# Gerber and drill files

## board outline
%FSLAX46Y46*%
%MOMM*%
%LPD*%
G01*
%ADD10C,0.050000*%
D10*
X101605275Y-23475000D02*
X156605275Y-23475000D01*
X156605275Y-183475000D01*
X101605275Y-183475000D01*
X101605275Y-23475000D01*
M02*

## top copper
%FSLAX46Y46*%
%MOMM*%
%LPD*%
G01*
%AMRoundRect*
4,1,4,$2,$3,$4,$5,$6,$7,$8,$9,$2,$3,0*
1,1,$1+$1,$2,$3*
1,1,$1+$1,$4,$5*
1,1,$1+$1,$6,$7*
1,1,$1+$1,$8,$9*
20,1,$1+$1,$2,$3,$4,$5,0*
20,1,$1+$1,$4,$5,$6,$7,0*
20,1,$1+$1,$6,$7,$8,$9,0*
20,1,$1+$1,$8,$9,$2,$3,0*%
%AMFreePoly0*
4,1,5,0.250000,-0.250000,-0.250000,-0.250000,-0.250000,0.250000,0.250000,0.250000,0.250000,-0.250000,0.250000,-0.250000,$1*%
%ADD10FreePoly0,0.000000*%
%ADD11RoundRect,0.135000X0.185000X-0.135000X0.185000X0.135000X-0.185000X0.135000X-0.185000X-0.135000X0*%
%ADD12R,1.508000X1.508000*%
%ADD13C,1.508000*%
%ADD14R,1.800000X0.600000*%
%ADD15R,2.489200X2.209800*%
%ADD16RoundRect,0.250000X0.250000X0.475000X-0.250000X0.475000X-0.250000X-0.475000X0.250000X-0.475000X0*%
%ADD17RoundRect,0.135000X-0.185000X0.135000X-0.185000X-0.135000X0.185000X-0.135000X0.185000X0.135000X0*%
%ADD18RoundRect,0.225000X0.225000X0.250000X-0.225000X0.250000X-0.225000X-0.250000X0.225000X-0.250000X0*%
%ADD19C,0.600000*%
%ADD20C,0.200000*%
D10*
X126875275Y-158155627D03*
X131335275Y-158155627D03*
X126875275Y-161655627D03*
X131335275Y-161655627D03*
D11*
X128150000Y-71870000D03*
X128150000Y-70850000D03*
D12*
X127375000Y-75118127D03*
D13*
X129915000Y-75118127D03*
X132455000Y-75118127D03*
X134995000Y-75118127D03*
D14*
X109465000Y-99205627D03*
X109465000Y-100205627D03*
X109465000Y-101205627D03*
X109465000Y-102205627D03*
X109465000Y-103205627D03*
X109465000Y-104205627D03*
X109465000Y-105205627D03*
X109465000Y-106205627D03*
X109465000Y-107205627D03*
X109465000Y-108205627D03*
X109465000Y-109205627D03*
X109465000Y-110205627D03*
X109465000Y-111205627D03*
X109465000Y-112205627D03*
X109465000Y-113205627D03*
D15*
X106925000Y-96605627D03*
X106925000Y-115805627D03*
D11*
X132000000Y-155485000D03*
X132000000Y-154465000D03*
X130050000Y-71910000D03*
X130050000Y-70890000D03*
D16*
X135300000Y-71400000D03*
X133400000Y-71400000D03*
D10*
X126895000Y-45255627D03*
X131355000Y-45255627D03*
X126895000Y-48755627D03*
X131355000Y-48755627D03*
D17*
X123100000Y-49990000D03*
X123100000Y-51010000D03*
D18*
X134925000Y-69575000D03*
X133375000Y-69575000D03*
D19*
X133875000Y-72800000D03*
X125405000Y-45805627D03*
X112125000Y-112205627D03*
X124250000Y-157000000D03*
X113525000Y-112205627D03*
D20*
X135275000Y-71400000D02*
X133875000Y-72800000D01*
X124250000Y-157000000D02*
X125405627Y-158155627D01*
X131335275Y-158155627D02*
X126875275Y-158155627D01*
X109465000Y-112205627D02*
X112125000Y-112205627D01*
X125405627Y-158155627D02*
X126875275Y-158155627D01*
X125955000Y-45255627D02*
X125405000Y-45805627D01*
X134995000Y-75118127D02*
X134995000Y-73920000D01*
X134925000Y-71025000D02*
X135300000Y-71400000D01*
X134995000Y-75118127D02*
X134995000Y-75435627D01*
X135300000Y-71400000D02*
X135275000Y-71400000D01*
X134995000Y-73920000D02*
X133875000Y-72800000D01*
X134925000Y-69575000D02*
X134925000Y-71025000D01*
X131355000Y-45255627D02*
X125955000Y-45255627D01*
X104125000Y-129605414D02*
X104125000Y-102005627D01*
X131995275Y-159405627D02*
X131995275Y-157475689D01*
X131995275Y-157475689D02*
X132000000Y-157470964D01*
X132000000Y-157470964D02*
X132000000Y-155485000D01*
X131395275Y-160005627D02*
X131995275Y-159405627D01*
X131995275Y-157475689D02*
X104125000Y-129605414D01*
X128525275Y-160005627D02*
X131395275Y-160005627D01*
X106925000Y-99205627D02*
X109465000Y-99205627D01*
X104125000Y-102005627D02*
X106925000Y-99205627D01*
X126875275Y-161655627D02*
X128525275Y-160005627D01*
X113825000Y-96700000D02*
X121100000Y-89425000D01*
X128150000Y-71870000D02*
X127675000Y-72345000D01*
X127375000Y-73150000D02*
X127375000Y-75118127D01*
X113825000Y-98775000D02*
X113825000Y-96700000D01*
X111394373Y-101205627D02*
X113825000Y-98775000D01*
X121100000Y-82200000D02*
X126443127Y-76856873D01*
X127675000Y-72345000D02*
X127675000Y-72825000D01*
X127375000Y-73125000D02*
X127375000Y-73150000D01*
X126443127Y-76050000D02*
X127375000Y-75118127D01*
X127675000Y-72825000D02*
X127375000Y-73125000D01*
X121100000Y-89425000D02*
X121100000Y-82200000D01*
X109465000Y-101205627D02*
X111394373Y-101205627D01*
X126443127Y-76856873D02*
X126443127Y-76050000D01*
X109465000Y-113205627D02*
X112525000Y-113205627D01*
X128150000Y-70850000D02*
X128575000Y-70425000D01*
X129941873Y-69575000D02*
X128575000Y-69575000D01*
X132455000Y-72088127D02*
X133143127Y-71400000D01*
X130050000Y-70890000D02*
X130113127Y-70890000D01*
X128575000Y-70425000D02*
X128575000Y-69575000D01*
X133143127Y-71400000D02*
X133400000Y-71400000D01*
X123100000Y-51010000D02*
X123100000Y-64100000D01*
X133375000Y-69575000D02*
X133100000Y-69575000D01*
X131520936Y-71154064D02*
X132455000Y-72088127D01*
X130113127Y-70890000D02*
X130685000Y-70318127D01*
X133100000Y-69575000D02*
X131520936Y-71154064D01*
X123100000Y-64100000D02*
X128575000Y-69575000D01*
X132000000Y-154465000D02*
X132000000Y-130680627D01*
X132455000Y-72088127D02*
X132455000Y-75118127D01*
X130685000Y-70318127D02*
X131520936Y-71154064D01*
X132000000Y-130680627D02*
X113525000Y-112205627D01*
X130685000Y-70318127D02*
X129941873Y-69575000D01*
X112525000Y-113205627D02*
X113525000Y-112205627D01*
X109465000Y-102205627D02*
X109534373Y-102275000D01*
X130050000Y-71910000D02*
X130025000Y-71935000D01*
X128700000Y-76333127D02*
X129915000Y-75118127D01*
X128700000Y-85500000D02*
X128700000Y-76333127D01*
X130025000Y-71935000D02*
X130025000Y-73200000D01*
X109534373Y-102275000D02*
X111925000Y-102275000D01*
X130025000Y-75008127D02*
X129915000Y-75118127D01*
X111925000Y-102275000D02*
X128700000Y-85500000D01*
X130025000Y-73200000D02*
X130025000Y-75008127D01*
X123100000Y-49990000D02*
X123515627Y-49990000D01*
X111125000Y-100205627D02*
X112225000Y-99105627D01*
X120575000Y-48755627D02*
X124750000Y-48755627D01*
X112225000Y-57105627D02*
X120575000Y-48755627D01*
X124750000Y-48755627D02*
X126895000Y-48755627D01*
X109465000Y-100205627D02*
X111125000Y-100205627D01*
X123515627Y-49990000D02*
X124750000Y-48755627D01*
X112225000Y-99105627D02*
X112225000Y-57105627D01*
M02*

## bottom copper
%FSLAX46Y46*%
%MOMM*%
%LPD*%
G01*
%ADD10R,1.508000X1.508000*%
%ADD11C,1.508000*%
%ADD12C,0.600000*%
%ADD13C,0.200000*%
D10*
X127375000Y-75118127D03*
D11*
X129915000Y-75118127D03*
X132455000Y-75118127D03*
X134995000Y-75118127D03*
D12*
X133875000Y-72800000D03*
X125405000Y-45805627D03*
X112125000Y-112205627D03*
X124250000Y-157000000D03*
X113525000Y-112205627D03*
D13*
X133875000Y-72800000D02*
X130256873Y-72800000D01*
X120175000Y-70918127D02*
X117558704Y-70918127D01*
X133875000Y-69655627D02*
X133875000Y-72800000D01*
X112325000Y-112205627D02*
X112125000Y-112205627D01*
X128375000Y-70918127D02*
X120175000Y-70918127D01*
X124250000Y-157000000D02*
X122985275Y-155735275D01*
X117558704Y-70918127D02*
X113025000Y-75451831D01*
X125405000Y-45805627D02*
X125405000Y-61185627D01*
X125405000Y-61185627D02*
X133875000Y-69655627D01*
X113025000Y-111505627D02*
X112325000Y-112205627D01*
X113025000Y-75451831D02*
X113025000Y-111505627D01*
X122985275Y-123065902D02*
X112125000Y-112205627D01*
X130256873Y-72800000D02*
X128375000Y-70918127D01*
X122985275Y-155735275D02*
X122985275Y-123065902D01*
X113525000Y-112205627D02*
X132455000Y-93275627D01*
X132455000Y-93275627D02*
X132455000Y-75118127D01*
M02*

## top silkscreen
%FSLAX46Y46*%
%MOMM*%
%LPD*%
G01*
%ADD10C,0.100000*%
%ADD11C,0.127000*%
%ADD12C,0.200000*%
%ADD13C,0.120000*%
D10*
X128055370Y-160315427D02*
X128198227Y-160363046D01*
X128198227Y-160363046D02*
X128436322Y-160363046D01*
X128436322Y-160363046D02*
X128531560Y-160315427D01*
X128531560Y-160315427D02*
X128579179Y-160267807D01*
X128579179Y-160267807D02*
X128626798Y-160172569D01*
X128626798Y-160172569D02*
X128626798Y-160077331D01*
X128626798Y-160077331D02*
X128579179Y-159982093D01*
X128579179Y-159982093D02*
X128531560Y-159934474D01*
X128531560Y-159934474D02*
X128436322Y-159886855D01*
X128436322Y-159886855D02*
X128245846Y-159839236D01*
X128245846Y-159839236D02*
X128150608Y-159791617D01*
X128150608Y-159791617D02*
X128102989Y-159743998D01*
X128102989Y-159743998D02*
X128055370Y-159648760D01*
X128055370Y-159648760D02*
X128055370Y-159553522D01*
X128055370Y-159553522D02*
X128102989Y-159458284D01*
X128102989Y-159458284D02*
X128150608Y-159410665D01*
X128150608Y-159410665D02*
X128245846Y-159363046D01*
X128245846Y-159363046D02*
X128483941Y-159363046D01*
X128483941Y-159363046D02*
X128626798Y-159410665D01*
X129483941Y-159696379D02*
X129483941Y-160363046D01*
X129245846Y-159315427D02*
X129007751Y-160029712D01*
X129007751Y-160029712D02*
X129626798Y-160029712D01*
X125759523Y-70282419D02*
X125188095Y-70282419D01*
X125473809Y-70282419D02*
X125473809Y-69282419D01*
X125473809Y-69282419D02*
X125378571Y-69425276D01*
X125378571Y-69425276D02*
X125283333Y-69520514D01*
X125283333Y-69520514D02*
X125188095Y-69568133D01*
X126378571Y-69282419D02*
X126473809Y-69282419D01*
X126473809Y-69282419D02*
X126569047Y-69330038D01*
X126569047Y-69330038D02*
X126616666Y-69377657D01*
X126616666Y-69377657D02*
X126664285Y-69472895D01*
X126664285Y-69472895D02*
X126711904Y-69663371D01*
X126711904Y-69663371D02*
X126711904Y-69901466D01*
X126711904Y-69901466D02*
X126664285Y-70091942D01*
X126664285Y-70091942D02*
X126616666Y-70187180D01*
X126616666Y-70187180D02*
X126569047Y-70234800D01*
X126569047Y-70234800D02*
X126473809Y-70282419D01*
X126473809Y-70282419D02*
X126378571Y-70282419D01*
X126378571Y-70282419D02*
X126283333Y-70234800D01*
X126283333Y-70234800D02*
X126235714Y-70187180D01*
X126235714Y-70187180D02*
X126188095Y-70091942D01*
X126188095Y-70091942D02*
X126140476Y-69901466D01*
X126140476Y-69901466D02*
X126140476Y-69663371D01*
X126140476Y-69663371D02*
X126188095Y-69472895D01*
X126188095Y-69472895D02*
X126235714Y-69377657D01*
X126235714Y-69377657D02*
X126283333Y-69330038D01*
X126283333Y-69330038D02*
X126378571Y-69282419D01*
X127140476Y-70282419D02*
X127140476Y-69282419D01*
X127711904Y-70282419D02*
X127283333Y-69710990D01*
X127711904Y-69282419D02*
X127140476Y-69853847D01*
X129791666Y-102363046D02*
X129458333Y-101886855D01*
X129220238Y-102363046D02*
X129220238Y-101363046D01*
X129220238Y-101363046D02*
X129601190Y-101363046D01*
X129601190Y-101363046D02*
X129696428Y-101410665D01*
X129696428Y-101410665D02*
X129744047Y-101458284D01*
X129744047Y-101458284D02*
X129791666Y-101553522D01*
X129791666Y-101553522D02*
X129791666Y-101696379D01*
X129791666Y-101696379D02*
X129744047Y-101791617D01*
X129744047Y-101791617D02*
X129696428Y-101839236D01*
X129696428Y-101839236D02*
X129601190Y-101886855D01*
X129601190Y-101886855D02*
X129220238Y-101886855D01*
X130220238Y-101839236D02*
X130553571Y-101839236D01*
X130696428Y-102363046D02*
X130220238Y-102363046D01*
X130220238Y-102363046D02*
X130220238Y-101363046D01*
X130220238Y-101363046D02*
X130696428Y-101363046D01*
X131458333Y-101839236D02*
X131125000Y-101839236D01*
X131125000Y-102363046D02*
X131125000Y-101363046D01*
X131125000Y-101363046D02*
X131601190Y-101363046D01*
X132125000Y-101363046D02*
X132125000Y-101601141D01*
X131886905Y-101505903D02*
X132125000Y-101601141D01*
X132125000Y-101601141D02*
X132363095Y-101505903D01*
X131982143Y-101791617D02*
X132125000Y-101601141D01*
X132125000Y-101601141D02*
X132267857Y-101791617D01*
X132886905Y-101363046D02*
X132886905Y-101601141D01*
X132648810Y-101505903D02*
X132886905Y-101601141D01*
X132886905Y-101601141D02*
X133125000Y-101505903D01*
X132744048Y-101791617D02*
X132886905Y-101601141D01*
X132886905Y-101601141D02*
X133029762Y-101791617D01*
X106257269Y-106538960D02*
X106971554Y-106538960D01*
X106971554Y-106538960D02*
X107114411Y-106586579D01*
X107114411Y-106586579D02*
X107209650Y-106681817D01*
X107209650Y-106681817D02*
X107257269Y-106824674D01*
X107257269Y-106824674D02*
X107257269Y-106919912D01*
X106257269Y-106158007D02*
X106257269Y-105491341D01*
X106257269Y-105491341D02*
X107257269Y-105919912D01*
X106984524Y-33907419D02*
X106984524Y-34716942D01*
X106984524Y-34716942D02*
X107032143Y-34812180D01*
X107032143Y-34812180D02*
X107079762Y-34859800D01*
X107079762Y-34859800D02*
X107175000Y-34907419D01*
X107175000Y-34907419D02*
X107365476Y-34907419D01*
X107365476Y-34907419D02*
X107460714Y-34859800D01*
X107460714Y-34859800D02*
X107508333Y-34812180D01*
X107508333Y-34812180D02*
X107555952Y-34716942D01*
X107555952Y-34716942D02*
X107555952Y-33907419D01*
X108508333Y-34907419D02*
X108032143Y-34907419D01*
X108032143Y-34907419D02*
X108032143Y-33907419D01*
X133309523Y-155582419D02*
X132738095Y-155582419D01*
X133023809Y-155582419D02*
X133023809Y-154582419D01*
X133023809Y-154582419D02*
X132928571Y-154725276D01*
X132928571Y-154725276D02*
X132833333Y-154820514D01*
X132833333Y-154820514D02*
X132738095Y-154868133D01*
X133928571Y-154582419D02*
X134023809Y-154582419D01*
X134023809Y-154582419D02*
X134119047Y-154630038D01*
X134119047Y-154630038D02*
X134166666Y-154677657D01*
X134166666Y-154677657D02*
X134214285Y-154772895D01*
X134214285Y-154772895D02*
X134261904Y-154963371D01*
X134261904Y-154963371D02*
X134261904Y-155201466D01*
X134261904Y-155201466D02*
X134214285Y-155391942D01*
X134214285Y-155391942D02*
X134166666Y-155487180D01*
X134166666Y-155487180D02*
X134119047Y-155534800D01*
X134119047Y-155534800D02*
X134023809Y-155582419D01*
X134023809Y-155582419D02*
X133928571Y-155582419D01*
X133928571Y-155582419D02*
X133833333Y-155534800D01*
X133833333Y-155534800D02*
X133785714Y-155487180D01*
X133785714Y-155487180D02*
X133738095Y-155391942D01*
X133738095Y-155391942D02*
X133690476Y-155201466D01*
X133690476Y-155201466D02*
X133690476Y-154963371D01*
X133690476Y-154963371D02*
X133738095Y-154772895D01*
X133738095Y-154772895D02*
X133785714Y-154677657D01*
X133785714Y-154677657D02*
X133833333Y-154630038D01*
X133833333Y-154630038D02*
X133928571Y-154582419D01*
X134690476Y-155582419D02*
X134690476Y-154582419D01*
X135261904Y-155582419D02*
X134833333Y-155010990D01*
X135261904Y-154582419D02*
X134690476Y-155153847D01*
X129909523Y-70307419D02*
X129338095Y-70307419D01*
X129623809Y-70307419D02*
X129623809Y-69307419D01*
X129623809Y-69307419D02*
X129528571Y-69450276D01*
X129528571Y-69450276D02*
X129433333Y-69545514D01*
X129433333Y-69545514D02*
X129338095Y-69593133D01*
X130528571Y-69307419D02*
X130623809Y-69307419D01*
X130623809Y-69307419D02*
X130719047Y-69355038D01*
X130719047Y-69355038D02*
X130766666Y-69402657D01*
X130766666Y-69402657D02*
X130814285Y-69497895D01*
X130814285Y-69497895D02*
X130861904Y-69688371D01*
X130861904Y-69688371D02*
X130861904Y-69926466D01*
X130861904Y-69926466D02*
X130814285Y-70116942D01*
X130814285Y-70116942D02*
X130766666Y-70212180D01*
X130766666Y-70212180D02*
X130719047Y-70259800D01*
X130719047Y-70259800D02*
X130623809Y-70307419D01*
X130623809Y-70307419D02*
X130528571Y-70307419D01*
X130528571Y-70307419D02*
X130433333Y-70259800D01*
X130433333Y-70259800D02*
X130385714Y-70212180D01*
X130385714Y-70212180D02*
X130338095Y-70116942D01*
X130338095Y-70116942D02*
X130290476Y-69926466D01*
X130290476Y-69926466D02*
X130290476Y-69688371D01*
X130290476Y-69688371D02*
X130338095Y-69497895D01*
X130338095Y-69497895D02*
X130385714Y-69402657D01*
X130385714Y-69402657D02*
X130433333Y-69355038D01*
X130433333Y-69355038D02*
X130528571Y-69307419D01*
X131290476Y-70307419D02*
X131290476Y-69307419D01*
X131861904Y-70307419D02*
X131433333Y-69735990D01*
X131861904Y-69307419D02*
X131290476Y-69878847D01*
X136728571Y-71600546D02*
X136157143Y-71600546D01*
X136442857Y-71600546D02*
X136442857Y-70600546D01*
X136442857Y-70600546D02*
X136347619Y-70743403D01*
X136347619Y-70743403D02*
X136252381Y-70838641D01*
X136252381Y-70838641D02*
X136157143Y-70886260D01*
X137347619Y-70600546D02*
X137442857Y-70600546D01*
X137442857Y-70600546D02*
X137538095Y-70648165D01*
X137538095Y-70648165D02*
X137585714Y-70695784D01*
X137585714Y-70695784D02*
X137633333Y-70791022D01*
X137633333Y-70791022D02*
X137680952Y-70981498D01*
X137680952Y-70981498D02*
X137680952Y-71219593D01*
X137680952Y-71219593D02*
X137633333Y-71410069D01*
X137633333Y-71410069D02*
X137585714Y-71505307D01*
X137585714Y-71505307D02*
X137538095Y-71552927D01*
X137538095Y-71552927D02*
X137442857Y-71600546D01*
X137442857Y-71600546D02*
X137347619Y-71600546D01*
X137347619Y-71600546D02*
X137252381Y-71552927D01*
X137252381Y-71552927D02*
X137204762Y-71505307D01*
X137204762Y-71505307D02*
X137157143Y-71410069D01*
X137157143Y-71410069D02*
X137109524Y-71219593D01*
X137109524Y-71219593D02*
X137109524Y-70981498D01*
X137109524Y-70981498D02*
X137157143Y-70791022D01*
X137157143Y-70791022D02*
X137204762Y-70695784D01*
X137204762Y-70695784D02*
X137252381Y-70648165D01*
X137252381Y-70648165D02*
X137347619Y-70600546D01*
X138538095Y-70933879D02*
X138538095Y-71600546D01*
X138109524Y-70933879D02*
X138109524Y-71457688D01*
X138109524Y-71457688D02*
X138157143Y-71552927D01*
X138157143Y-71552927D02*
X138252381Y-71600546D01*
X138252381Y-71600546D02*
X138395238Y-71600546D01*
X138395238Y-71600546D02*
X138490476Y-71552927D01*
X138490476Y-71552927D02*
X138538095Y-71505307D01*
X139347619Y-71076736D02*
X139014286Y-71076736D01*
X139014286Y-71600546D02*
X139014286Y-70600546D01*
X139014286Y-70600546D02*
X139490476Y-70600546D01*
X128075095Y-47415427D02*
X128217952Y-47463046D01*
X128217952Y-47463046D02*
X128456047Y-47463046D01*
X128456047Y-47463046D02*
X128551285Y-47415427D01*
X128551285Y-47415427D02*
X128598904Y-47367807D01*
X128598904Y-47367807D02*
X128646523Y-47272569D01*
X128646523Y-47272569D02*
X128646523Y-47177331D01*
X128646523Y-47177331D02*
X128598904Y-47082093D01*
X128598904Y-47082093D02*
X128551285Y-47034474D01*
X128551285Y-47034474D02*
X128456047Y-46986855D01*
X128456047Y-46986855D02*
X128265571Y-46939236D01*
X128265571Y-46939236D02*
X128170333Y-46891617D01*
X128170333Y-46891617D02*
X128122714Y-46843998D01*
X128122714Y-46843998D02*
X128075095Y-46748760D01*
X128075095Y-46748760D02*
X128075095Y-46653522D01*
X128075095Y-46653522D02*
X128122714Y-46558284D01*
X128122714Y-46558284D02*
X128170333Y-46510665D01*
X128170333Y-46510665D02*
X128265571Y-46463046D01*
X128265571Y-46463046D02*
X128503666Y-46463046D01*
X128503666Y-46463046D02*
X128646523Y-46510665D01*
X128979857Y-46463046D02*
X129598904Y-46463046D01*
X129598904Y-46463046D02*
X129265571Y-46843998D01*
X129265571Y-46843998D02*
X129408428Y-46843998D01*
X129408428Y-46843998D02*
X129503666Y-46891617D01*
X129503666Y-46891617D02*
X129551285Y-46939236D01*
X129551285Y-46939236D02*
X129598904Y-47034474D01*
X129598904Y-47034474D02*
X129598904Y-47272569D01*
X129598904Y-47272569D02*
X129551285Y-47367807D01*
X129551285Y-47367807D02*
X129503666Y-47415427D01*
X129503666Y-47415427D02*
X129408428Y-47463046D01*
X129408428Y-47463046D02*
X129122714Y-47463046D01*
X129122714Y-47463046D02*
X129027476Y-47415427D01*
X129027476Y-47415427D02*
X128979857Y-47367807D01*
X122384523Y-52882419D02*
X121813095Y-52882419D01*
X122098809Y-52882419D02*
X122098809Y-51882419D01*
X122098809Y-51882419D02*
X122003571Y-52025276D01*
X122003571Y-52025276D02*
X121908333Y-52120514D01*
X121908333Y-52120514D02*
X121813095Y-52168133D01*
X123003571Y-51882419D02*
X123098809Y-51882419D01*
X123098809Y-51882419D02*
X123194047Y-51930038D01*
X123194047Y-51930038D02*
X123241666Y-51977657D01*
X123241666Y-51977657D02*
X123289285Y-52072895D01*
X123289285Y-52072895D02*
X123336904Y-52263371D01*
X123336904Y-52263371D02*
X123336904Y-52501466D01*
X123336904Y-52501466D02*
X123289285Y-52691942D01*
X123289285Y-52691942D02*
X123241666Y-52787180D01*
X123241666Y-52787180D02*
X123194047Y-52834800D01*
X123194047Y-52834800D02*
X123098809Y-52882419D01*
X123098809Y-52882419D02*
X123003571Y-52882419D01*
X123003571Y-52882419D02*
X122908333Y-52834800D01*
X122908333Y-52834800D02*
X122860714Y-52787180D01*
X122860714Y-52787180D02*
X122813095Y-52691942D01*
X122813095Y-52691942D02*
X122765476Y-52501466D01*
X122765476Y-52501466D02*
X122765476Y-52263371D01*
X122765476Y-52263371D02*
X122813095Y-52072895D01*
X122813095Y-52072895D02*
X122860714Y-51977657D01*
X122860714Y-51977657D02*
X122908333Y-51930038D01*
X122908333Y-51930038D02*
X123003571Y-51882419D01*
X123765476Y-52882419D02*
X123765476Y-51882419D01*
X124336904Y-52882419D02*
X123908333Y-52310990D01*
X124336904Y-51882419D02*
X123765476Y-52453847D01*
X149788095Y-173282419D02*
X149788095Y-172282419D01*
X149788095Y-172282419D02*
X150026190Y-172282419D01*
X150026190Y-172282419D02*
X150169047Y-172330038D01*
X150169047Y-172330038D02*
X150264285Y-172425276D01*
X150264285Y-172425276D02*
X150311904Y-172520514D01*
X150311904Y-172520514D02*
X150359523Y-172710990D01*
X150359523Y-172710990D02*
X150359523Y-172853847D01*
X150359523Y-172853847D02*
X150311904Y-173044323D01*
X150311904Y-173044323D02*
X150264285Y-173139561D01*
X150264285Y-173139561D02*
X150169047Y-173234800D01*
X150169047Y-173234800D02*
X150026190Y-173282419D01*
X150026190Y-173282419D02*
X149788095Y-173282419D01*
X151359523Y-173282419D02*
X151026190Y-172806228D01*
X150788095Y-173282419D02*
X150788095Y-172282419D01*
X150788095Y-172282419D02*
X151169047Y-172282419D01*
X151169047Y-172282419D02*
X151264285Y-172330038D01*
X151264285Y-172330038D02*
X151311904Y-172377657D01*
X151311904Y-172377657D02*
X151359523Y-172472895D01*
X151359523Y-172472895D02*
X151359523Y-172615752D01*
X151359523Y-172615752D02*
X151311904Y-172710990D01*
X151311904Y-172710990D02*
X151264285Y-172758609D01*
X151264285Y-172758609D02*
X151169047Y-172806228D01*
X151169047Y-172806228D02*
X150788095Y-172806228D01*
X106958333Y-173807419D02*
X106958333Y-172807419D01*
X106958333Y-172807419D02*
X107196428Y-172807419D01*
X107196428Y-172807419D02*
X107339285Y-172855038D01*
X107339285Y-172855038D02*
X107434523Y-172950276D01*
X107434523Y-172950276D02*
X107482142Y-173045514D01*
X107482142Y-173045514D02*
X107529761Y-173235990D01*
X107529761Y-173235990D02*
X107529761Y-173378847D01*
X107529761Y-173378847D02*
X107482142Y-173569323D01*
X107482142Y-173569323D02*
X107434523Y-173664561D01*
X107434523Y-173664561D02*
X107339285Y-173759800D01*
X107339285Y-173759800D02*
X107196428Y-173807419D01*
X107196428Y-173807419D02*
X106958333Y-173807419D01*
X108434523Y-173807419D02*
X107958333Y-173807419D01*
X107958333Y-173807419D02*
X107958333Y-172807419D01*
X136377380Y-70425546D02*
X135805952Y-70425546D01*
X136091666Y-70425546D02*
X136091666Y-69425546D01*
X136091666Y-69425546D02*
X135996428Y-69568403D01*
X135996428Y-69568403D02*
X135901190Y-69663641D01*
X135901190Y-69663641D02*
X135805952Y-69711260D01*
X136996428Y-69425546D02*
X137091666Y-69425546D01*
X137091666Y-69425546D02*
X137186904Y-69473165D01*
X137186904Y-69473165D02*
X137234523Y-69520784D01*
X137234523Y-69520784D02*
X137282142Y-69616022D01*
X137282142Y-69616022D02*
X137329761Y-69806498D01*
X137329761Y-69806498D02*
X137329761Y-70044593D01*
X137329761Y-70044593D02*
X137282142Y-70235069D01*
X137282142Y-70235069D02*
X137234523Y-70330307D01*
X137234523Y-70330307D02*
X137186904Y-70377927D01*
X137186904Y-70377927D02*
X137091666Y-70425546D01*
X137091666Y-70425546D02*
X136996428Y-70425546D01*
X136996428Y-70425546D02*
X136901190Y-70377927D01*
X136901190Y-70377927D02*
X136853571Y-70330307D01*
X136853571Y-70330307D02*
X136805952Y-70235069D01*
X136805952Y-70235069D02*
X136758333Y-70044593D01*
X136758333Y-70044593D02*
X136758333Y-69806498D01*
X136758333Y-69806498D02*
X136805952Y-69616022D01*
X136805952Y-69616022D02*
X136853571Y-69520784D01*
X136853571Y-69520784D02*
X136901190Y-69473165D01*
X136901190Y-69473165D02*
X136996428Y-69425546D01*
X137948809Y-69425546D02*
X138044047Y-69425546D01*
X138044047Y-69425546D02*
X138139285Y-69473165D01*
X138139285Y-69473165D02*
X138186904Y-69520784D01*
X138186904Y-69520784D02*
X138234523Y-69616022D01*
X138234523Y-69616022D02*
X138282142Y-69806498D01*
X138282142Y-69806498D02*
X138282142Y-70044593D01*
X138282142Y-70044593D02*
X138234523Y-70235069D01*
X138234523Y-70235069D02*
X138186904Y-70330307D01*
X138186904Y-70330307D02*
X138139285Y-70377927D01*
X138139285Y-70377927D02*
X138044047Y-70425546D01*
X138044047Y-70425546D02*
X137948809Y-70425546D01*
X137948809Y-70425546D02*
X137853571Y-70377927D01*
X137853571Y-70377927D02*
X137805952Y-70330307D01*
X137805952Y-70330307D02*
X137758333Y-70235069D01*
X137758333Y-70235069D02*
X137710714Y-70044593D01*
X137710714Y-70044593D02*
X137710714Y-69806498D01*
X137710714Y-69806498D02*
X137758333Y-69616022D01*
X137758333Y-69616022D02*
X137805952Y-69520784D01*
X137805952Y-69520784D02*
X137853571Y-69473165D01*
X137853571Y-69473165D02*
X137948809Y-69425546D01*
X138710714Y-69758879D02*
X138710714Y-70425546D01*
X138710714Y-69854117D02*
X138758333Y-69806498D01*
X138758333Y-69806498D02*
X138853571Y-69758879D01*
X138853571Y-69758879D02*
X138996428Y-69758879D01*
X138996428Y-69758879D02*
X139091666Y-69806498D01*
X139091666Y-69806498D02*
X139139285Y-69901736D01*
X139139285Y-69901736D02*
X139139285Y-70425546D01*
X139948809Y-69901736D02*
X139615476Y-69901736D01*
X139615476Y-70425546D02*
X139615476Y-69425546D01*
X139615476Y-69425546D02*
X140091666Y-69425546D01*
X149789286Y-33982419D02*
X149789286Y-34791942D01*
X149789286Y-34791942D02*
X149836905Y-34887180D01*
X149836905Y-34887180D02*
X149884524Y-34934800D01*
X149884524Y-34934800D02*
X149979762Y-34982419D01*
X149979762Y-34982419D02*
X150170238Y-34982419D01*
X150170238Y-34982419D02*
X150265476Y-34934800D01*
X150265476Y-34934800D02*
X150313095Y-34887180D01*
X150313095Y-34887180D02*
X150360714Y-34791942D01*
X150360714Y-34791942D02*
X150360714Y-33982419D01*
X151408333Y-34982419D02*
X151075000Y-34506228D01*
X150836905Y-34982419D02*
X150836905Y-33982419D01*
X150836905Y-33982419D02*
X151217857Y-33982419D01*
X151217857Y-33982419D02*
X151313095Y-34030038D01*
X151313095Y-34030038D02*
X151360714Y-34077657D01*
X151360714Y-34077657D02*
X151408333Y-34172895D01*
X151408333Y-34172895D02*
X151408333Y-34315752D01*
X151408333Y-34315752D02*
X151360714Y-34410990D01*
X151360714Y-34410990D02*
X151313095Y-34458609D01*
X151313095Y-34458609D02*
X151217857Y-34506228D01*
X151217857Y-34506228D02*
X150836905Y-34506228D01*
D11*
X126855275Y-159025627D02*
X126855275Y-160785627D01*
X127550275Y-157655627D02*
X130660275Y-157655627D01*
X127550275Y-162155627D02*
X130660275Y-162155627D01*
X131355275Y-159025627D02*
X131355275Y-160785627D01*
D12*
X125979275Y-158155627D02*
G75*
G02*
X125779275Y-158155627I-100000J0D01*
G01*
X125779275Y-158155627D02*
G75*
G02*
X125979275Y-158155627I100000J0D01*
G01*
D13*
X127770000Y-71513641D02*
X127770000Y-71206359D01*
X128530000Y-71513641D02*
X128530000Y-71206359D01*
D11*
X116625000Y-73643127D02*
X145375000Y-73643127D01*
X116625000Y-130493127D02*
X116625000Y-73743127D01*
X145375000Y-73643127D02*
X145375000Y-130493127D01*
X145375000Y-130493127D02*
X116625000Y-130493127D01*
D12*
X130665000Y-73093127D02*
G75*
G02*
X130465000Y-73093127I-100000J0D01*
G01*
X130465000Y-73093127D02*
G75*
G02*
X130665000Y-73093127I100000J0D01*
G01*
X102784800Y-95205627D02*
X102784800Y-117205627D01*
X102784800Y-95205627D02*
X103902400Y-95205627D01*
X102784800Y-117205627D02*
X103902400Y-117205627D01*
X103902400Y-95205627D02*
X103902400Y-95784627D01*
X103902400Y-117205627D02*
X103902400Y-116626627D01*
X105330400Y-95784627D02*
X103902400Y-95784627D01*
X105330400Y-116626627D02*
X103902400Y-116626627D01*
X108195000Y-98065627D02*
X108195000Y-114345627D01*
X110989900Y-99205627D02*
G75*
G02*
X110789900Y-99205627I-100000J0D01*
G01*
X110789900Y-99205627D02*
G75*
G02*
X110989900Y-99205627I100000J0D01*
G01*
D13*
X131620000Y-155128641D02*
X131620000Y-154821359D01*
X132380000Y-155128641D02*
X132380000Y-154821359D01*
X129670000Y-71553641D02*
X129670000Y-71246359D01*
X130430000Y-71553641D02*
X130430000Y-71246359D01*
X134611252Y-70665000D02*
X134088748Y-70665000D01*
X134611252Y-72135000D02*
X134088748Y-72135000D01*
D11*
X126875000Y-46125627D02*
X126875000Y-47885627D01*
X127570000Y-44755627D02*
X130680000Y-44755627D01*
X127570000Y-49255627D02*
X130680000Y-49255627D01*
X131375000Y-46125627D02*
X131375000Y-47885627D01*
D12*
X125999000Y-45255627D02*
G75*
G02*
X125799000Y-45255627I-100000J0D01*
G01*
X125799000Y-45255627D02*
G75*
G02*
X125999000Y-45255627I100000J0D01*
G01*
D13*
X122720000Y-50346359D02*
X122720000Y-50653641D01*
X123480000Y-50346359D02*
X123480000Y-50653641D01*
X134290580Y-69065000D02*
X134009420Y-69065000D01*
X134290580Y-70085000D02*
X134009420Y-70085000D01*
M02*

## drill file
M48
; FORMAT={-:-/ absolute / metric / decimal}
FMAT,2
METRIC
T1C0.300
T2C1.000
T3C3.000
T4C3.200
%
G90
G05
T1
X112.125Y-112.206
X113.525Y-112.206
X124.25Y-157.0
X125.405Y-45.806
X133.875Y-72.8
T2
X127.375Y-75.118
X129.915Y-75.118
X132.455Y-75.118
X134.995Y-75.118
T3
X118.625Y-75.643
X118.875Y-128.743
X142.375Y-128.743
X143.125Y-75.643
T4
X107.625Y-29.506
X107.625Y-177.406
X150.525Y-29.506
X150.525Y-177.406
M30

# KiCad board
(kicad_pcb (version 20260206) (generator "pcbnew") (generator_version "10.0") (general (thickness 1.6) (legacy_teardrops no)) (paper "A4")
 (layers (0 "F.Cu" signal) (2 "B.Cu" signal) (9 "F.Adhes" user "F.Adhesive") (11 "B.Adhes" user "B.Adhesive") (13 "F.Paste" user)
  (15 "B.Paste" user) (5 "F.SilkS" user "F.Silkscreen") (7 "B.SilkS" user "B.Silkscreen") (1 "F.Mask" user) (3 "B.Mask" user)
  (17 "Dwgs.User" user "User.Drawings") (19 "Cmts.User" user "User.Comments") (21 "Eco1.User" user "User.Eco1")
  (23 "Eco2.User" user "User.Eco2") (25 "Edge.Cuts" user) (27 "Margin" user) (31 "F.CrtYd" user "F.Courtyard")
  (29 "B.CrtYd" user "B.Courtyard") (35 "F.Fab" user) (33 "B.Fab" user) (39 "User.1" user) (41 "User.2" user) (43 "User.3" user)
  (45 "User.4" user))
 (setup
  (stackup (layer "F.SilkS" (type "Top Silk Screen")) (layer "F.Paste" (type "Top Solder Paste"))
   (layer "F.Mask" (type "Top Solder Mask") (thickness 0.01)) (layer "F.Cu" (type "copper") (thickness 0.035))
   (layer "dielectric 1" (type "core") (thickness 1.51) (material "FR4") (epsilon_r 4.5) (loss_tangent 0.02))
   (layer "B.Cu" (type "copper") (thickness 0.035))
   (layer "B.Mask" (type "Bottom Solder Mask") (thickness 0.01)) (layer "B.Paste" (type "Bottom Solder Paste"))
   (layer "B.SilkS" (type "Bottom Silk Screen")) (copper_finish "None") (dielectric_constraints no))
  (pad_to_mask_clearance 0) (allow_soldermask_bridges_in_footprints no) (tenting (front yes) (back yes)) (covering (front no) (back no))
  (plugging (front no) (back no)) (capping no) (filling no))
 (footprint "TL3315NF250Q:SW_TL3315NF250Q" (layer "F.Cu") (at 129.105275 159.905627)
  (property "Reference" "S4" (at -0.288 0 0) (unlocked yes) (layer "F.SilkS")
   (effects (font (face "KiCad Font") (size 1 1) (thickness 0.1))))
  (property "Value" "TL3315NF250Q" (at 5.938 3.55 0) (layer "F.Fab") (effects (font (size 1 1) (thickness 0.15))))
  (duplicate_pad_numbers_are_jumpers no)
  (fp_line (start -2.25 -0.88) (end -2.25 0.88) (stroke (width 0.127) (type solid)) (layer "F.SilkS"))
  (fp_line (start -1.555 -2.25) (end 1.555 -2.25) (stroke (width 0.127) (type solid)) (layer "F.SilkS"))
  (fp_line (start -1.555 2.25) (end 1.555 2.25) (stroke (width 0.127) (type solid)) (layer "F.SilkS"))
  (fp_line (start 2.25 -0.88) (end 2.25 0.88) (stroke (width 0.127) (type solid)) (layer "F.SilkS"))
  (fp_circle (center -3.226 -1.75) (end -3.126 -1.75) (stroke (width 0.2) (type solid)) (fill no) (layer "F.SilkS"))
  (pad "1" smd custom (at -2.23 -1.75) (size 0.5 0.5) (layers "F.Cu") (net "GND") (options (clearance outline) (anchor rect)) (primitives))
  (pad "2" smd custom (at 2.23 -1.75) (size 0.5 0.5) (layers "F.Cu") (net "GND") (options (clearance outline) (anchor rect)) (primitives))
  (pad "3" smd custom (at -2.23 1.75) (size 0.5 0.5) (layers "F.Cu") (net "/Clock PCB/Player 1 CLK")
   (options (clearance outline) (anchor rect)) (primitives))
  (pad "4" smd custom (at 2.23 1.75) (size 0.5 0.5) (layers "F.Cu") (options (clearance outline) (anchor rect)) (primitives)))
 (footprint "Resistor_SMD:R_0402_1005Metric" (layer "F.Cu") (at 128.15 71.36 90)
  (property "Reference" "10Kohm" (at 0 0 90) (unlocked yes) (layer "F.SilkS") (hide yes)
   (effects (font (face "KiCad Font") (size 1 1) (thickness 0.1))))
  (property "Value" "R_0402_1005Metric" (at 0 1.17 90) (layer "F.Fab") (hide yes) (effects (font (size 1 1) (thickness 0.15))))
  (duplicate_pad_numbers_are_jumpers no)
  (fp_line (start -0.153641 -0.38) (end 0.153641 -0.38) (stroke (width 0.12) (type solid)) (layer "F.SilkS"))
  (fp_line (start -0.153641 0.38) (end 0.153641 0.38) (stroke (width 0.12) (type solid)) (layer "F.SilkS"))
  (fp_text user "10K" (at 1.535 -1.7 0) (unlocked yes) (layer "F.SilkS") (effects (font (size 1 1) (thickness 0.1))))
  (pad "1" smd roundrect (at -0.51 0 90) (size 0.54 0.64) (layers "F.Cu" "F.Mask" "F.Paste") (roundrect_rratio 0.25) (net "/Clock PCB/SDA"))
  (pad "2" smd roundrect (at 0.51 0 90) (size 0.54 0.64) (layers "F.Cu" "F.Mask" "F.Paste") (roundrect_rratio 0.25) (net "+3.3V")))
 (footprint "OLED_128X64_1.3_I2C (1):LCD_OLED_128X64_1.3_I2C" (layer "F.Cu") (at 131.125 101.368127)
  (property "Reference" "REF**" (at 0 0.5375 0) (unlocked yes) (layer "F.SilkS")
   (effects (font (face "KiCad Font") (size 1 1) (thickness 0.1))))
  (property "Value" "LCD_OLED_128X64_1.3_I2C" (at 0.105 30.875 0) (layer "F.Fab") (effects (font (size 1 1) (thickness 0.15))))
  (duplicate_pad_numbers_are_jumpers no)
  (fp_line (start -14.5 -27.725) (end 14.25 -27.725) (stroke (width 0.127) (type solid)) (layer "F.SilkS"))
  (fp_line (start -14.5 29.125) (end -14.5 -27.625) (stroke (width 0.127) (type solid)) (layer "F.SilkS"))
  (fp_line (start 14.25 -27.725) (end 14.25 29.125) (stroke (width 0.127) (type solid)) (layer "F.SilkS"))
  (fp_line (start 14.25 29.125) (end -14.5 29.125) (stroke (width 0.127) (type solid)) (layer "F.SilkS"))
  (fp_circle (center -0.56 -28.275) (end -0.46 -28.275) (stroke (width 0.2) (type solid)) (fill no) (layer "F.SilkS"))
  (pad "" np_thru_hole circle (at -12.5 -25.725) (size 3 3) (drill 3) (layers "*.Cu" "*.Mask"))
  (pad "" np_thru_hole circle (at -12.25 27.375) (size 3 3) (drill 3) (layers "*.Cu" "*.Mask"))
  (pad "" np_thru_hole circle (at 11.25 27.375) (size 3 3) (drill 3) (layers "*.Cu" "*.Mask"))
  (pad "" np_thru_hole circle (at 12 -25.725) (size 3 3) (drill 3) (layers "*.Cu" "*.Mask"))
  (pad "1" thru_hole rect (at -3.75 -26.25) (size 1.508 1.508) (drill 1) (layers "*.Cu" "*.Mask") (remove_unused_layers no)
   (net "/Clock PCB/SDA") (solder_mask_margin 0.102))
  (pad "2" thru_hole circle (at -1.21 -26.25) (size 1.508 1.508) (drill 1) (layers "*.Cu" "*.Mask") (remove_unused_layers no)
   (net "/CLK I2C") (solder_mask_margin 0.102))
  (pad "3" thru_hole circle (at 1.33 -26.25) (size 1.508 1.508) (drill 1) (layers "*.Cu" "*.Mask") (remove_unused_layers no) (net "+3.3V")
   (solder_mask_margin 0.102))
  (pad "4" thru_hole circle (at 3.87 -26.25) (size 1.508 1.508) (drill 1) (layers "*.Cu" "*.Mask") (remove_unused_layers no) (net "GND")
   (solder_mask_margin 0.102)))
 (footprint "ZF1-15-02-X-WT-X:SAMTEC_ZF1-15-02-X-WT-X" (layer "F.Cu") (at 105.4899 106.205627 -90)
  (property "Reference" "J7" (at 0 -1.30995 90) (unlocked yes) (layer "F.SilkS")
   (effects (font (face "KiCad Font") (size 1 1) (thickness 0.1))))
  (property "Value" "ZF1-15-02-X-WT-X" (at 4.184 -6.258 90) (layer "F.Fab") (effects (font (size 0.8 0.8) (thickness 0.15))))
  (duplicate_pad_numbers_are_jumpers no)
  (fp_line (start -11 2.7051) (end 11 2.7051) (stroke (width 0.2) (type solid)) (layer "F.SilkS"))
  (fp_line (start -11 2.7051) (end -11 1.5875) (stroke (width 0.2) (type solid)) (layer "F.SilkS"))
  (fp_line (start 11 2.7051) (end 11 1.5875) (stroke (width 0.2) (type solid)) (layer "F.SilkS"))
  (fp_line (start -11 1.5875) (end -10.421 1.5875) (stroke (width 0.2) (type solid)) (layer "F.SilkS"))
  (fp_line (start 11 1.5875) (end 10.421 1.5875) (stroke (width 0.2) (type solid)) (layer "F.SilkS"))
  (fp_line (start -10.421 0.1595) (end -10.421 1.5875) (stroke (width 0.2) (type solid)) (layer "F.SilkS"))
  (fp_line (start 10.421 0.1595) (end 10.421 1.5875) (stroke (width 0.2) (type solid)) (layer "F.SilkS"))
  (fp_line (start -8.14 -2.7051) (end 8.14 -2.7051) (stroke (width 0.2) (type solid)) (layer "F.SilkS"))
  (fp_circle (center -7 -5.4) (end -6.9 -5.4) (stroke (width 0.2) (type solid)) (fill no) (layer "F.SilkS"))
  (pad "01" smd rect (at -7 -3.9751 270) (size 0.6 1.8) (layers "F.Cu" "F.Mask" "F.Paste") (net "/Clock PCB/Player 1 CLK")
   (solder_mask_margin 0.102))
  (pad "02" smd rect (at -6 -3.9751 270) (size 0.6 1.8) (layers "F.Cu" "F.Mask" "F.Paste") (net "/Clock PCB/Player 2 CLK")
   (solder_mask_margin 0.102))
  (pad "03" smd rect (at -5 -3.9751 270) (size 0.6 1.8) (layers "F.Cu" "F.Mask" "F.Paste") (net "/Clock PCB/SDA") (solder_mask_margin 0.102))
  (pad "04" smd rect (at -4 -3.9751 270) (size 0.6 1.8) (layers "F.Cu" "F.Mask" "F.Paste") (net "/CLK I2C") (solder_mask_margin 0.102))
  (pad "05" smd rect (at -3 -3.9751 270) (size 0.6 1.8) (layers "F.Cu" "F.Mask" "F.Paste") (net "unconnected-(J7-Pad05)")
   (solder_mask_margin 0.102))
  (pad "06" smd rect (at -2 -3.9751 270) (size 0.6 1.8) (layers "F.Cu" "F.Mask" "F.Paste") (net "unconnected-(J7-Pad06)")
   (solder_mask_margin 0.102))
  (pad "07" smd rect (at -1 -3.9751 270) (size 0.6 1.8) (layers "F.Cu" "F.Mask" "F.Paste") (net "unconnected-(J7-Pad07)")
   (solder_mask_margin 0.102))
  (pad "08" smd rect (at 0 -3.9751 270) (size 0.6 1.8) (layers "F.Cu" "F.Mask" "F.Paste") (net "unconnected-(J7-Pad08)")
   (solder_mask_margin 0.102))
  (pad "09" smd rect (at 1 -3.9751 270) (size 0.6 1.8) (layers "F.Cu" "F.Mask" "F.Paste") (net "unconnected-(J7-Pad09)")
   (solder_mask_margin 0.102))
  (pad "10" smd rect (at 2 -3.9751 270) (size 0.6 1.8) (layers "F.Cu" "F.Mask" "F.Paste") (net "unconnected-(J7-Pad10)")
   (solder_mask_margin 0.102))
  (pad "11" smd rect (at 3 -3.9751 270) (size 0.6 1.8) (layers "F.Cu" "F.Mask" "F.Paste") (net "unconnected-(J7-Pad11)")
   (solder_mask_margin 0.102))
  (pad "12" smd rect (at 4 -3.9751 270) (size 0.6 1.8) (layers "F.Cu" "F.Mask" "F.Paste") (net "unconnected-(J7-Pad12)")
   (solder_mask_margin 0.102))
  (pad "13" smd rect (at 5 -3.9751 270) (size 0.6 1.8) (layers "F.Cu" "F.Mask" "F.Paste") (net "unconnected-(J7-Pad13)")
   (solder_mask_margin 0.102))
  (pad "14" smd rect (at 6 -3.9751 270) (size 0.6 1.8) (layers "F.Cu" "F.Mask" "F.Paste") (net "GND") (solder_mask_margin 0.102))
  (pad "15" smd rect (at 7 -3.9751 270) (size 0.6 1.8) (layers "F.Cu" "F.Mask" "F.Paste") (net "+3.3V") (solder_mask_margin 0.102))
  (pad "MP1" smd rect (at -9.6 -1.4351 270) (size 2.2098 2.4892) (layers "F.Cu" "F.Mask" "F.Paste") (solder_mask_margin 0.102))
  (pad "MP2" smd rect (at 9.6 -1.4351 270) (size 2.2098 2.4892) (layers "F.Cu" "F.Mask" "F.Paste") (solder_mask_margin 0.102)))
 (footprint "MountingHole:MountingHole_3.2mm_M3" (layer "F.Cu") (at 107.625 29.505627)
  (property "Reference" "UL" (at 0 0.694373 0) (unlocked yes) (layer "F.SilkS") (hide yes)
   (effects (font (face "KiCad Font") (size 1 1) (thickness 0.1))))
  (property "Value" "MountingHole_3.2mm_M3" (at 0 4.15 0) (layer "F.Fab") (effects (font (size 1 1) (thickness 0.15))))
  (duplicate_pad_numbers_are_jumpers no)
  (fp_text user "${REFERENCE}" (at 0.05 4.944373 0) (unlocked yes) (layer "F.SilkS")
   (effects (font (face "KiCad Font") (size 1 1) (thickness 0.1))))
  (pad "" np_thru_hole circle (at 0 0) (size 3.2 3.2) (drill 3.2) (layers "*.Cu" "*.Mask")))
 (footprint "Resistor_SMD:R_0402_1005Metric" (layer "F.Cu") (at 132 154.975 90)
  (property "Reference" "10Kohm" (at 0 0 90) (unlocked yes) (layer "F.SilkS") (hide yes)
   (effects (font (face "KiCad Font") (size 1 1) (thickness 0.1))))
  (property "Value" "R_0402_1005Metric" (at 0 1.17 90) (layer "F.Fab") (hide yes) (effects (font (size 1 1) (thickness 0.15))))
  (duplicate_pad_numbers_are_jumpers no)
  (fp_line (start -0.153641 -0.38) (end 0.153641 -0.38) (stroke (width 0.12) (type solid)) (layer "F.SilkS"))
  (fp_line (start -0.153641 0.38) (end 0.153641 0.38) (stroke (width 0.12) (type solid)) (layer "F.SilkS"))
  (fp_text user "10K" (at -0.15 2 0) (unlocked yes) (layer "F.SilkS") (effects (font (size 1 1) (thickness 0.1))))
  (pad "1" smd roundrect (at -0.51 0 90) (size 0.54 0.64) (layers "F.Cu" "F.Mask" "F.Paste") (roundrect_rratio 0.25)
   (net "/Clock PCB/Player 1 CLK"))
  (pad "2" smd roundrect (at 0.51 0 90) (size 0.54 0.64) (layers "F.Cu" "F.Mask" "F.Paste") (roundrect_rratio 0.25) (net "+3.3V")))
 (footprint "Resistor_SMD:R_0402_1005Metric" (layer "F.Cu") (at 130.05 71.4 90)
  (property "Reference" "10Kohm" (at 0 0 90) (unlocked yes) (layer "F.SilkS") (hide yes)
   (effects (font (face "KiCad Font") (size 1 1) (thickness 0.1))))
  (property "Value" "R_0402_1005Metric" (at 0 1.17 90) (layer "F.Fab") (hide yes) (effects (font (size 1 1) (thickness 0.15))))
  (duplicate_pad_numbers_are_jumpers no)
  (fp_line (start -0.153641 -0.38) (end 0.153641 -0.38) (stroke (width 0.12) (type solid)) (layer "F.SilkS"))
  (fp_line (start -0.153641 0.38) (end 0.153641 0.38) (stroke (width 0.12) (type solid)) (layer "F.SilkS"))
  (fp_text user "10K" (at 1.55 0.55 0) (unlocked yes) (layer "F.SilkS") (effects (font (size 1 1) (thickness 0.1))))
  (pad "1" smd roundrect (at -0.51 0 90) (size 0.54 0.64) (layers "F.Cu" "F.Mask" "F.Paste") (roundrect_rratio 0.25) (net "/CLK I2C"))
  (pad "2" smd roundrect (at 0.51 0 90) (size 0.54 0.64) (layers "F.Cu" "F.Mask" "F.Paste") (roundrect_rratio 0.25) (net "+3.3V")))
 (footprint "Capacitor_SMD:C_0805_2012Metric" (layer "F.Cu") (at 134.35 71.4 180)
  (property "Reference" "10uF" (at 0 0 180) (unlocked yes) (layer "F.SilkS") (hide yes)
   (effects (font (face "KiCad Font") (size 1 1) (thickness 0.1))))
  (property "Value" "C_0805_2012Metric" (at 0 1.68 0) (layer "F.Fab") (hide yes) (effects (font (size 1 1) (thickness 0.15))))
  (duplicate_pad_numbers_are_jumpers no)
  (fp_line (start -0.261252 0.735) (end 0.261252 0.735) (stroke (width 0.12) (type solid)) (layer "F.SilkS"))
  (fp_line (start -0.261252 -0.735) (end 0.261252 -0.735) (stroke (width 0.12) (type solid)) (layer "F.SilkS"))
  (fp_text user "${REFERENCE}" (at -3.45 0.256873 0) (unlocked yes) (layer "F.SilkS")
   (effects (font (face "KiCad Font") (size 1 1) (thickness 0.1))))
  (pad "1" smd roundrect (at -0.95 0 180) (size 1 1.45) (layers "F.Cu" "F.Mask" "F.Paste") (roundrect_rratio 0.25) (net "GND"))
  (pad "2" smd roundrect (at 0.95 0 180) (size 1 1.45) (layers "F.Cu" "F.Mask" "F.Paste") (roundrect_rratio 0.25) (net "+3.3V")))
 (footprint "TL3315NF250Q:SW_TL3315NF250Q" (layer "F.Cu") (at 129.125 47.005627)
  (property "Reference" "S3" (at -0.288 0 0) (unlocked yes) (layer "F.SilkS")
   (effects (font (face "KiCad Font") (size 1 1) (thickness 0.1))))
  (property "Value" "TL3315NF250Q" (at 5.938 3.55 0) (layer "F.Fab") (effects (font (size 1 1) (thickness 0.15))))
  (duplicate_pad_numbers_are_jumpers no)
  (fp_line (start -2.25 -0.88) (end -2.25 0.88) (stroke (width 0.127) (type solid)) (layer "F.SilkS"))
  (fp_line (start -1.555 -2.25) (end 1.555 -2.25) (stroke (width 0.127) (type solid)) (layer "F.SilkS"))
  (fp_line (start -1.555 2.25) (end 1.555 2.25) (stroke (width 0.127) (type solid)) (layer "F.SilkS"))
  (fp_line (start 2.25 -0.88) (end 2.25 0.88) (stroke (width 0.127) (type solid)) (layer "F.SilkS"))
  (fp_circle (center -3.226 -1.75) (end -3.126 -1.75) (stroke (width 0.2) (type solid)) (fill no) (layer "F.SilkS"))
  (pad "1" smd custom (at -2.23 -1.75) (size 0.5 0.5) (layers "F.Cu") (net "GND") (options (clearance outline) (anchor rect)) (primitives))
  (pad "2" smd custom (at 2.23 -1.75) (size 0.5 0.5) (layers "F.Cu") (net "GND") (options (clearance outline) (anchor rect)) (primitives))
  (pad "3" smd custom (at -2.23 1.75) (size 0.5 0.5) (layers "F.Cu") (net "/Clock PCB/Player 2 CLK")
   (options (clearance outline) (anchor rect)) (primitives))
  (pad "4" smd custom (at 2.23 1.75) (size 0.5 0.5) (layers "F.Cu") (options (clearance outline) (anchor rect)) (primitives)))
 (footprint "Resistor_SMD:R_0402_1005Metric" (layer "F.Cu") (at 123.1 50.5 -90)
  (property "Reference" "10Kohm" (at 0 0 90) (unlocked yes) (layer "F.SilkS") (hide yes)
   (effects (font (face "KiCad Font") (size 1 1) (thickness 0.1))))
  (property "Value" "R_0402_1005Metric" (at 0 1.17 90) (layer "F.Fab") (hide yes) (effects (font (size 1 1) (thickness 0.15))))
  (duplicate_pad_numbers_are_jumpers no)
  (fp_line (start -0.153641 0.38) (end 0.153641 0.38) (stroke (width 0.12) (type solid)) (layer "F.SilkS"))
  (fp_line (start -0.153641 -0.38) (end 0.153641 -0.38) (stroke (width 0.12) (type solid)) (layer "F.SilkS"))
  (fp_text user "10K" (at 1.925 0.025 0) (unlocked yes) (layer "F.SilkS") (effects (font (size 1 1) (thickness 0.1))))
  (pad "1" smd roundrect (at -0.51 0 270) (size 0.54 0.64) (layers "F.Cu" "F.Mask" "F.Paste") (roundrect_rratio 0.25)
   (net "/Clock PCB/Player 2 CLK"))
  (pad "2" smd roundrect (at 0.51 0 270) (size 0.54 0.64) (layers "F.Cu" "F.Mask" "F.Paste") (roundrect_rratio 0.25) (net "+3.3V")))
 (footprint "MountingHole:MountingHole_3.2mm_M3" (layer "F.Cu") (at 150.525 177.405627)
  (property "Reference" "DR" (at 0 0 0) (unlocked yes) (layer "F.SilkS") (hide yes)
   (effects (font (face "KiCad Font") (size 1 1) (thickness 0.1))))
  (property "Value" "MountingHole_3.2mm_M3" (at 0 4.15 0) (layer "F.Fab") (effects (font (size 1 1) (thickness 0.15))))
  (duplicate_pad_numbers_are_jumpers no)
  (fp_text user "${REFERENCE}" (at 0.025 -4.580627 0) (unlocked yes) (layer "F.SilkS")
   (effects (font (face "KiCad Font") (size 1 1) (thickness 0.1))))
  (pad "" np_thru_hole circle (at 0 0) (size 3.2 3.2) (drill 3.2) (layers "*.Cu" "*.Mask")))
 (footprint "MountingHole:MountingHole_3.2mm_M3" (layer "F.Cu") (at 107.625 177.405627)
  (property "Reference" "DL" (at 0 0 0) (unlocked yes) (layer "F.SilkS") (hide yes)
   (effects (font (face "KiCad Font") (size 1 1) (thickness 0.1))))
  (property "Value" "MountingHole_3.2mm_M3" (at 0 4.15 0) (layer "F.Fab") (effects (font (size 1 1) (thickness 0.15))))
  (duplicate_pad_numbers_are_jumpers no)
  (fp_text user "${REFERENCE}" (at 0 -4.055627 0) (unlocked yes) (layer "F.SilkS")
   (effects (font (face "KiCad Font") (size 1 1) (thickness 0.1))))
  (pad "" np_thru_hole circle (at 0 0) (size 3.2 3.2) (drill 3.2) (layers "*.Cu" "*.Mask")))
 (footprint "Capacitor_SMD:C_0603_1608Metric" (layer "F.Cu") (at 134.15 69.575 180)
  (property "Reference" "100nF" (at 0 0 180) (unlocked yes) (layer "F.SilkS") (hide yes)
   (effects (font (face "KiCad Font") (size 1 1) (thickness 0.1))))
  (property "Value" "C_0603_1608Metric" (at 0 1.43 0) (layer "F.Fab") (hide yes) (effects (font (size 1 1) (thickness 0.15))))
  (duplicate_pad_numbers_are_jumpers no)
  (fp_line (start -0.14058 0.51) (end 0.14058 0.51) (stroke (width 0.12) (type solid)) (layer "F.SilkS"))
  (fp_line (start -0.14058 -0.51) (end 0.14058 -0.51) (stroke (width 0.12) (type solid)) (layer "F.SilkS"))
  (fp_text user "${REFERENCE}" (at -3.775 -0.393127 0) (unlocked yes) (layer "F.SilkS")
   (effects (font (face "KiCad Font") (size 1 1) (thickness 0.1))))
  (pad "1" smd roundrect (at -0.775 0 180) (size 0.9 0.95) (layers "F.Cu" "F.Mask" "F.Paste") (roundrect_rratio 0.25) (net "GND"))
  (pad "2" smd roundrect (at 0.775 0 180) (size 0.9 0.95) (layers "F.Cu" "F.Mask" "F.Paste") (roundrect_rratio 0.25) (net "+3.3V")))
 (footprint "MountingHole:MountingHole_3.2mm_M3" (layer "F.Cu") (at 150.525 29.505627)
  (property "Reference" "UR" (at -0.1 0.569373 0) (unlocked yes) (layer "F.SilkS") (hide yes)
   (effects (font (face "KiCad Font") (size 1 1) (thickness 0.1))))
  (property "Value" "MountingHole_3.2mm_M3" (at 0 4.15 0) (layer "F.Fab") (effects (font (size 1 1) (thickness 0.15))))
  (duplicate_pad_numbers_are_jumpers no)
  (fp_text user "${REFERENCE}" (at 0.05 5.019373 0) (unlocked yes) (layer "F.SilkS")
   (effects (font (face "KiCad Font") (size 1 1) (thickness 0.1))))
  (pad "" np_thru_hole circle (at 0 0) (size 3.2 3.2) (drill 3.2) (layers "*.Cu" "*.Mask")))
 (gr_rect (start 101.605275 23.475) (end 156.605275 183.475) (stroke (width 0.05) (type solid)) (fill no) (layer "Edge.Cuts"))
 (segment (start 135.275 71.4) (end 133.875 72.8) (width 0.2) (layer "F.Cu") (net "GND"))
 (segment (start 124.25 157) (end 125.405627 158.155627) (width 0.2) (layer "F.Cu") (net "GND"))
 (segment (start 131.335275 158.155627) (end 126.875275 158.155627) (width 0.2) (layer "F.Cu") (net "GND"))
 (segment (start 109.465 112.205627) (end 112.125 112.205627) (width 0.2) (layer "F.Cu") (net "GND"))
 (segment (start 125.405627 158.155627) (end 126.875275 158.155627) (width 0.2) (layer "F.Cu") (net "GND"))
 (segment (start 125.955 45.255627) (end 125.405 45.805627) (width 0.2) (layer "F.Cu") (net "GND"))
 (segment (start 134.995 75.118127) (end 134.995 73.92) (width 0.2) (layer "F.Cu") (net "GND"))
 (segment (start 134.925 71.025) (end 135.3 71.4) (width 0.2) (layer "F.Cu") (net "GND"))
 (segment (start 134.995 75.118127) (end 134.995 75.435627) (width 0.2) (layer "F.Cu") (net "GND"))
 (segment (start 135.3 71.4) (end 135.275 71.4) (width 0.2) (layer "F.Cu") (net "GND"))
 (segment (start 134.995 73.92) (end 133.875 72.8) (width 0.2) (layer "F.Cu") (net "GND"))
 (segment (start 134.925 69.575) (end 134.925 71.025) (width 0.2) (layer "F.Cu") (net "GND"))
 (segment (start 131.355 45.255627) (end 125.955 45.255627) (width 0.2) (layer "F.Cu") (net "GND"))
 (via (at 133.875 72.8) (size 0.6) (drill 0.3) (layers "F.Cu" "B.Cu") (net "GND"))
 (via (at 125.405 45.805627) (size 0.6) (drill 0.3) (layers "F.Cu" "B.Cu") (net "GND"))
 (via (at 112.125 112.205627) (size 0.6) (drill 0.3) (layers "F.Cu" "B.Cu") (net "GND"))
 (via (at 124.25 157) (size 0.6) (drill 0.3) (layers "F.Cu" "B.Cu") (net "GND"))
 (segment (start 133.875 72.8) (end 130.256873 72.8) (width 0.2) (layer "B.Cu") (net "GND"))
 (segment (start 120.175 70.918127) (end 117.558704 70.918127) (width 0.2) (layer "B.Cu") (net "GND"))
 (segment (start 133.875 69.655627) (end 133.875 72.8) (width 0.2) (layer "B.Cu") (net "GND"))
 (segment (start 112.325 112.205627) (end 112.125 112.205627) (width 0.2) (layer "B.Cu") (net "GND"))
 (segment (start 128.375 70.918127) (end 120.175 70.918127) (width 0.2) (layer "B.Cu") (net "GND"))
 (segment (start 124.25 157) (end 122.985275 155.735275) (width 0.2) (layer "B.Cu") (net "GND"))
 (segment (start 117.558704 70.918127) (end 113.025 75.451831) (width 0.2) (layer "B.Cu") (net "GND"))
 (segment (start 125.405 45.805627) (end 125.405 61.185627) (width 0.2) (layer "B.Cu") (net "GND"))
 (segment (start 125.405 61.185627) (end 133.875 69.655627) (width 0.2) (layer "B.Cu") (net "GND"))
 (segment (start 113.025 111.505627) (end 112.325 112.205627) (width 0.2) (layer "B.Cu") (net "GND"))
 (segment (start 113.025 75.451831) (end 113.025 111.505627) (width 0.2) (layer "B.Cu") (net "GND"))
 (segment (start 122.985275 123.065902) (end 112.125 112.205627) (width 0.2) (layer "B.Cu") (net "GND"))
 (segment (start 130.256873 72.8) (end 128.375 70.918127) (width 0.2) (layer "B.Cu") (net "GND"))
 (segment (start 122.985275 155.735275) (end 122.985275 123.065902) (width 0.2) (layer "B.Cu") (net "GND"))
 (segment (start 104.125 129.605414) (end 104.125 102.005627) (width 0.2) (layer "F.Cu") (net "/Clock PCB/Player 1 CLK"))
 (segment (start 131.995275 159.405627) (end 131.995275 157.475689) (width 0.2) (layer "F.Cu") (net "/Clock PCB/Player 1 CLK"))
 (segment (start 131.995275 157.475689) (end 132 157.470964) (width 0.2) (layer "F.Cu") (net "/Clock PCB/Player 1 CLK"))
 (segment (start 132 157.470964) (end 132 155.485) (width 0.2) (layer "F.Cu") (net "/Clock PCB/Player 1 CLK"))
 (segment (start 131.395275 160.005627) (end 131.995275 159.405627) (width 0.2) (layer "F.Cu") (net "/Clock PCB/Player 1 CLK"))
 (segment (start 131.995275 157.475689) (end 104.125 129.605414) (width 0.2) (layer "F.Cu") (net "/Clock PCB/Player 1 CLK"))
 (segment (start 128.525275 160.005627) (end 131.395275 160.005627) (width 0.2) (layer "F.Cu") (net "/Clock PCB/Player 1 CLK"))
 (segment (start 106.925 99.205627) (end 109.465 99.205627) (width 0.2) (layer "F.Cu") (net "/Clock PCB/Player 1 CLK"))
 (segment (start 104.125 102.005627) (end 106.925 99.205627) (width 0.2) (layer "F.Cu") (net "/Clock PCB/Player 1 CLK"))
 (segment (start 126.875275 161.655627) (end 128.525275 160.005627) (width 0.2) (layer "F.Cu") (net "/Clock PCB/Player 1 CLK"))
 (segment (start 113.825 96.7) (end 121.1 89.425) (width 0.2) (layer "F.Cu") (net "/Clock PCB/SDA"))
 (segment (start 128.15 71.87) (end 127.675 72.345) (width 0.2) (layer "F.Cu") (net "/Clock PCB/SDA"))
 (segment (start 127.375 73.15) (end 127.375 75.118127) (width 0.2) (layer "F.Cu") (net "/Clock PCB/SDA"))
 (segment (start 113.825 98.775) (end 113.825 96.7) (width 0.2) (layer "F.Cu") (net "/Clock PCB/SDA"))
 (segment (start 111.394373 101.205627) (end 113.825 98.775) (width 0.2) (layer "F.Cu") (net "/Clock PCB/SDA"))
 (segment (start 121.1 82.2) (end 126.443127 76.856873) (width 0.2) (layer "F.Cu") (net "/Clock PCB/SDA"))
 (segment (start 127.675 72.345) (end 127.675 72.825) (width 0.2) (layer "F.Cu") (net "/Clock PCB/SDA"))
 (segment (start 127.375 73.125) (end 127.375 73.15) (width 0.2) (layer "F.Cu") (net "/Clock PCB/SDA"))
 (segment (start 126.443127 76.05) (end 127.375 75.118127) (width 0.2) (layer "F.Cu") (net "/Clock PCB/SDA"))
 (segment (start 127.675 72.825) (end 127.375 73.125) (width 0.2) (layer "F.Cu") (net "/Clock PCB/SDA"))
 (segment (start 121.1 89.425) (end 121.1 82.2) (width 0.2) (layer "F.Cu") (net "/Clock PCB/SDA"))
 (segment (start 109.465 101.205627) (end 111.394373 101.205627) (width 0.2) (layer "F.Cu") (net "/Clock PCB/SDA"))
 (segment (start 126.443127 76.856873) (end 126.443127 76.05) (width 0.2) (layer "F.Cu") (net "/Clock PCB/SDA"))
 (segment (start 109.465 113.205627) (end 112.525 113.205627) (width 0.2) (layer "F.Cu") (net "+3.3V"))
 (segment (start 128.15 70.85) (end 128.575 70.425) (width 0.2) (layer "F.Cu") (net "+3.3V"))
 (segment (start 129.941873 69.575) (end 128.575 69.575) (width 0.2) (layer "F.Cu") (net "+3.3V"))
 (segment (start 132.455 72.088127) (end 133.143127 71.4) (width 0.2) (layer "F.Cu") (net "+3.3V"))
 (segment (start 130.05 70.89) (end 130.113127 70.89) (width 0.2) (layer "F.Cu") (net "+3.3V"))
 (segment (start 128.575 70.425) (end 128.575 69.575) (width 0.2) (layer "F.Cu") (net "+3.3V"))
 (segment (start 133.143127 71.4) (end 133.4 71.4) (width 0.2) (layer "F.Cu") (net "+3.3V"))
 (segment (start 123.1 51.01) (end 123.1 64.1) (width 0.2) (layer "F.Cu") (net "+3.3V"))
 (segment (start 133.375 69.575) (end 133.1 69.575) (width 0.2) (layer "F.Cu") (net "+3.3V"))
 (segment (start 131.520936 71.154064) (end 132.455 72.088127) (width 0.2) (layer "F.Cu") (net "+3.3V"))
 (segment (start 130.113127 70.89) (end 130.685 70.318127) (width 0.2) (layer "F.Cu") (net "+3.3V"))
 (segment (start 133.1 69.575) (end 131.520936 71.154064) (width 0.2) (layer "F.Cu") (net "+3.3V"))
 (segment (start 123.1 64.1) (end 128.575 69.575) (width 0.2) (layer "F.Cu") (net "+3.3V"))
 (segment (start 132 154.465) (end 132 130.680627) (width 0.2) (layer "F.Cu") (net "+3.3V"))
 (segment (start 132.455 72.088127) (end 132.455 75.118127) (width 0.2) (layer "F.Cu") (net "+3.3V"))
 (segment (start 130.685 70.318127) (end 131.520936 71.154064) (width 0.2) (layer "F.Cu") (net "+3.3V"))
 (segment (start 132 130.680627) (end 113.525 112.205627) (width 0.2) (layer "F.Cu") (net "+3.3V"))
 (segment (start 130.685 70.318127) (end 129.941873 69.575) (width 0.2) (layer "F.Cu") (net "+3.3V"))
 (segment (start 112.525 113.205627) (end 113.525 112.205627) (width 0.2) (layer "F.Cu") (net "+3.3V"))
 (via (at 113.525 112.205627) (size 0.6) (drill 0.3) (layers "F.Cu" "B.Cu") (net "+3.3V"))
 (segment (start 113.525 112.205627) (end 132.455 93.275627) (width 0.2) (layer "B.Cu") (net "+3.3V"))
 (segment (start 132.455 93.275627) (end 132.455 75.118127) (width 0.2) (layer "B.Cu") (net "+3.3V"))
 (segment (start 109.465 102.205627) (end 109.534373 102.275) (width 0.2) (layer "F.Cu") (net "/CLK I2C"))
 (segment (start 130.05 71.91) (end 130.025 71.935) (width 0.2) (layer "F.Cu") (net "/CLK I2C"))
 (segment (start 128.7 76.333127) (end 129.915 75.118127) (width 0.2) (layer "F.Cu") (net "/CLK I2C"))
 (segment (start 128.7 85.5) (end 128.7 76.333127) (width 0.2) (layer "F.Cu") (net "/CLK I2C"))
 (segment (start 130.025 71.935) (end 130.025 73.2) (width 0.2) (layer "F.Cu") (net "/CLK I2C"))
 (segment (start 109.534373 102.275) (end 111.925 102.275) (width 0.2) (layer "F.Cu") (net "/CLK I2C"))
 (segment (start 130.025 75.008127) (end 129.915 75.118127) (width 0.2) (layer "F.Cu") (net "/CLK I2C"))
 (segment (start 111.925 102.275) (end 128.7 85.5) (width 0.2) (layer "F.Cu") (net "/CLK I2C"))
 (segment (start 130.025 73.2) (end 130.025 75.008127) (width 0.2) (layer "F.Cu") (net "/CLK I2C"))
 (segment (start 123.1 49.99) (end 123.515627 49.99) (width 0.2) (layer "F.Cu") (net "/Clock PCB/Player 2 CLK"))
 (segment (start 111.125 100.205627) (end 112.225 99.105627) (width 0.2) (layer "F.Cu") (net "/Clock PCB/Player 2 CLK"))
 (segment (start 120.575 48.755627) (end 124.75 48.755627) (width 0.2) (layer "F.Cu") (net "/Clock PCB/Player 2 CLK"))
 (segment (start 112.225 57.105627) (end 120.575 48.755627) (width 0.2) (layer "F.Cu") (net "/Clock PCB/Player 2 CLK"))
 (segment (start 124.75 48.755627) (end 126.895 48.755627) (width 0.2) (layer "F.Cu") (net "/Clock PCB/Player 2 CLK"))
 (segment (start 109.465 100.205627) (end 111.125 100.205627) (width 0.2) (layer "F.Cu") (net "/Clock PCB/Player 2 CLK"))
 (segment (start 123.515627 49.99) (end 124.75 48.755627) (width 0.2) (layer "F.Cu") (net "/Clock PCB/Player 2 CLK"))
 (segment (start 112.225 99.105627) (end 112.225 57.105627) (width 0.2) (layer "F.Cu") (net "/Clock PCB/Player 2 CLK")))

